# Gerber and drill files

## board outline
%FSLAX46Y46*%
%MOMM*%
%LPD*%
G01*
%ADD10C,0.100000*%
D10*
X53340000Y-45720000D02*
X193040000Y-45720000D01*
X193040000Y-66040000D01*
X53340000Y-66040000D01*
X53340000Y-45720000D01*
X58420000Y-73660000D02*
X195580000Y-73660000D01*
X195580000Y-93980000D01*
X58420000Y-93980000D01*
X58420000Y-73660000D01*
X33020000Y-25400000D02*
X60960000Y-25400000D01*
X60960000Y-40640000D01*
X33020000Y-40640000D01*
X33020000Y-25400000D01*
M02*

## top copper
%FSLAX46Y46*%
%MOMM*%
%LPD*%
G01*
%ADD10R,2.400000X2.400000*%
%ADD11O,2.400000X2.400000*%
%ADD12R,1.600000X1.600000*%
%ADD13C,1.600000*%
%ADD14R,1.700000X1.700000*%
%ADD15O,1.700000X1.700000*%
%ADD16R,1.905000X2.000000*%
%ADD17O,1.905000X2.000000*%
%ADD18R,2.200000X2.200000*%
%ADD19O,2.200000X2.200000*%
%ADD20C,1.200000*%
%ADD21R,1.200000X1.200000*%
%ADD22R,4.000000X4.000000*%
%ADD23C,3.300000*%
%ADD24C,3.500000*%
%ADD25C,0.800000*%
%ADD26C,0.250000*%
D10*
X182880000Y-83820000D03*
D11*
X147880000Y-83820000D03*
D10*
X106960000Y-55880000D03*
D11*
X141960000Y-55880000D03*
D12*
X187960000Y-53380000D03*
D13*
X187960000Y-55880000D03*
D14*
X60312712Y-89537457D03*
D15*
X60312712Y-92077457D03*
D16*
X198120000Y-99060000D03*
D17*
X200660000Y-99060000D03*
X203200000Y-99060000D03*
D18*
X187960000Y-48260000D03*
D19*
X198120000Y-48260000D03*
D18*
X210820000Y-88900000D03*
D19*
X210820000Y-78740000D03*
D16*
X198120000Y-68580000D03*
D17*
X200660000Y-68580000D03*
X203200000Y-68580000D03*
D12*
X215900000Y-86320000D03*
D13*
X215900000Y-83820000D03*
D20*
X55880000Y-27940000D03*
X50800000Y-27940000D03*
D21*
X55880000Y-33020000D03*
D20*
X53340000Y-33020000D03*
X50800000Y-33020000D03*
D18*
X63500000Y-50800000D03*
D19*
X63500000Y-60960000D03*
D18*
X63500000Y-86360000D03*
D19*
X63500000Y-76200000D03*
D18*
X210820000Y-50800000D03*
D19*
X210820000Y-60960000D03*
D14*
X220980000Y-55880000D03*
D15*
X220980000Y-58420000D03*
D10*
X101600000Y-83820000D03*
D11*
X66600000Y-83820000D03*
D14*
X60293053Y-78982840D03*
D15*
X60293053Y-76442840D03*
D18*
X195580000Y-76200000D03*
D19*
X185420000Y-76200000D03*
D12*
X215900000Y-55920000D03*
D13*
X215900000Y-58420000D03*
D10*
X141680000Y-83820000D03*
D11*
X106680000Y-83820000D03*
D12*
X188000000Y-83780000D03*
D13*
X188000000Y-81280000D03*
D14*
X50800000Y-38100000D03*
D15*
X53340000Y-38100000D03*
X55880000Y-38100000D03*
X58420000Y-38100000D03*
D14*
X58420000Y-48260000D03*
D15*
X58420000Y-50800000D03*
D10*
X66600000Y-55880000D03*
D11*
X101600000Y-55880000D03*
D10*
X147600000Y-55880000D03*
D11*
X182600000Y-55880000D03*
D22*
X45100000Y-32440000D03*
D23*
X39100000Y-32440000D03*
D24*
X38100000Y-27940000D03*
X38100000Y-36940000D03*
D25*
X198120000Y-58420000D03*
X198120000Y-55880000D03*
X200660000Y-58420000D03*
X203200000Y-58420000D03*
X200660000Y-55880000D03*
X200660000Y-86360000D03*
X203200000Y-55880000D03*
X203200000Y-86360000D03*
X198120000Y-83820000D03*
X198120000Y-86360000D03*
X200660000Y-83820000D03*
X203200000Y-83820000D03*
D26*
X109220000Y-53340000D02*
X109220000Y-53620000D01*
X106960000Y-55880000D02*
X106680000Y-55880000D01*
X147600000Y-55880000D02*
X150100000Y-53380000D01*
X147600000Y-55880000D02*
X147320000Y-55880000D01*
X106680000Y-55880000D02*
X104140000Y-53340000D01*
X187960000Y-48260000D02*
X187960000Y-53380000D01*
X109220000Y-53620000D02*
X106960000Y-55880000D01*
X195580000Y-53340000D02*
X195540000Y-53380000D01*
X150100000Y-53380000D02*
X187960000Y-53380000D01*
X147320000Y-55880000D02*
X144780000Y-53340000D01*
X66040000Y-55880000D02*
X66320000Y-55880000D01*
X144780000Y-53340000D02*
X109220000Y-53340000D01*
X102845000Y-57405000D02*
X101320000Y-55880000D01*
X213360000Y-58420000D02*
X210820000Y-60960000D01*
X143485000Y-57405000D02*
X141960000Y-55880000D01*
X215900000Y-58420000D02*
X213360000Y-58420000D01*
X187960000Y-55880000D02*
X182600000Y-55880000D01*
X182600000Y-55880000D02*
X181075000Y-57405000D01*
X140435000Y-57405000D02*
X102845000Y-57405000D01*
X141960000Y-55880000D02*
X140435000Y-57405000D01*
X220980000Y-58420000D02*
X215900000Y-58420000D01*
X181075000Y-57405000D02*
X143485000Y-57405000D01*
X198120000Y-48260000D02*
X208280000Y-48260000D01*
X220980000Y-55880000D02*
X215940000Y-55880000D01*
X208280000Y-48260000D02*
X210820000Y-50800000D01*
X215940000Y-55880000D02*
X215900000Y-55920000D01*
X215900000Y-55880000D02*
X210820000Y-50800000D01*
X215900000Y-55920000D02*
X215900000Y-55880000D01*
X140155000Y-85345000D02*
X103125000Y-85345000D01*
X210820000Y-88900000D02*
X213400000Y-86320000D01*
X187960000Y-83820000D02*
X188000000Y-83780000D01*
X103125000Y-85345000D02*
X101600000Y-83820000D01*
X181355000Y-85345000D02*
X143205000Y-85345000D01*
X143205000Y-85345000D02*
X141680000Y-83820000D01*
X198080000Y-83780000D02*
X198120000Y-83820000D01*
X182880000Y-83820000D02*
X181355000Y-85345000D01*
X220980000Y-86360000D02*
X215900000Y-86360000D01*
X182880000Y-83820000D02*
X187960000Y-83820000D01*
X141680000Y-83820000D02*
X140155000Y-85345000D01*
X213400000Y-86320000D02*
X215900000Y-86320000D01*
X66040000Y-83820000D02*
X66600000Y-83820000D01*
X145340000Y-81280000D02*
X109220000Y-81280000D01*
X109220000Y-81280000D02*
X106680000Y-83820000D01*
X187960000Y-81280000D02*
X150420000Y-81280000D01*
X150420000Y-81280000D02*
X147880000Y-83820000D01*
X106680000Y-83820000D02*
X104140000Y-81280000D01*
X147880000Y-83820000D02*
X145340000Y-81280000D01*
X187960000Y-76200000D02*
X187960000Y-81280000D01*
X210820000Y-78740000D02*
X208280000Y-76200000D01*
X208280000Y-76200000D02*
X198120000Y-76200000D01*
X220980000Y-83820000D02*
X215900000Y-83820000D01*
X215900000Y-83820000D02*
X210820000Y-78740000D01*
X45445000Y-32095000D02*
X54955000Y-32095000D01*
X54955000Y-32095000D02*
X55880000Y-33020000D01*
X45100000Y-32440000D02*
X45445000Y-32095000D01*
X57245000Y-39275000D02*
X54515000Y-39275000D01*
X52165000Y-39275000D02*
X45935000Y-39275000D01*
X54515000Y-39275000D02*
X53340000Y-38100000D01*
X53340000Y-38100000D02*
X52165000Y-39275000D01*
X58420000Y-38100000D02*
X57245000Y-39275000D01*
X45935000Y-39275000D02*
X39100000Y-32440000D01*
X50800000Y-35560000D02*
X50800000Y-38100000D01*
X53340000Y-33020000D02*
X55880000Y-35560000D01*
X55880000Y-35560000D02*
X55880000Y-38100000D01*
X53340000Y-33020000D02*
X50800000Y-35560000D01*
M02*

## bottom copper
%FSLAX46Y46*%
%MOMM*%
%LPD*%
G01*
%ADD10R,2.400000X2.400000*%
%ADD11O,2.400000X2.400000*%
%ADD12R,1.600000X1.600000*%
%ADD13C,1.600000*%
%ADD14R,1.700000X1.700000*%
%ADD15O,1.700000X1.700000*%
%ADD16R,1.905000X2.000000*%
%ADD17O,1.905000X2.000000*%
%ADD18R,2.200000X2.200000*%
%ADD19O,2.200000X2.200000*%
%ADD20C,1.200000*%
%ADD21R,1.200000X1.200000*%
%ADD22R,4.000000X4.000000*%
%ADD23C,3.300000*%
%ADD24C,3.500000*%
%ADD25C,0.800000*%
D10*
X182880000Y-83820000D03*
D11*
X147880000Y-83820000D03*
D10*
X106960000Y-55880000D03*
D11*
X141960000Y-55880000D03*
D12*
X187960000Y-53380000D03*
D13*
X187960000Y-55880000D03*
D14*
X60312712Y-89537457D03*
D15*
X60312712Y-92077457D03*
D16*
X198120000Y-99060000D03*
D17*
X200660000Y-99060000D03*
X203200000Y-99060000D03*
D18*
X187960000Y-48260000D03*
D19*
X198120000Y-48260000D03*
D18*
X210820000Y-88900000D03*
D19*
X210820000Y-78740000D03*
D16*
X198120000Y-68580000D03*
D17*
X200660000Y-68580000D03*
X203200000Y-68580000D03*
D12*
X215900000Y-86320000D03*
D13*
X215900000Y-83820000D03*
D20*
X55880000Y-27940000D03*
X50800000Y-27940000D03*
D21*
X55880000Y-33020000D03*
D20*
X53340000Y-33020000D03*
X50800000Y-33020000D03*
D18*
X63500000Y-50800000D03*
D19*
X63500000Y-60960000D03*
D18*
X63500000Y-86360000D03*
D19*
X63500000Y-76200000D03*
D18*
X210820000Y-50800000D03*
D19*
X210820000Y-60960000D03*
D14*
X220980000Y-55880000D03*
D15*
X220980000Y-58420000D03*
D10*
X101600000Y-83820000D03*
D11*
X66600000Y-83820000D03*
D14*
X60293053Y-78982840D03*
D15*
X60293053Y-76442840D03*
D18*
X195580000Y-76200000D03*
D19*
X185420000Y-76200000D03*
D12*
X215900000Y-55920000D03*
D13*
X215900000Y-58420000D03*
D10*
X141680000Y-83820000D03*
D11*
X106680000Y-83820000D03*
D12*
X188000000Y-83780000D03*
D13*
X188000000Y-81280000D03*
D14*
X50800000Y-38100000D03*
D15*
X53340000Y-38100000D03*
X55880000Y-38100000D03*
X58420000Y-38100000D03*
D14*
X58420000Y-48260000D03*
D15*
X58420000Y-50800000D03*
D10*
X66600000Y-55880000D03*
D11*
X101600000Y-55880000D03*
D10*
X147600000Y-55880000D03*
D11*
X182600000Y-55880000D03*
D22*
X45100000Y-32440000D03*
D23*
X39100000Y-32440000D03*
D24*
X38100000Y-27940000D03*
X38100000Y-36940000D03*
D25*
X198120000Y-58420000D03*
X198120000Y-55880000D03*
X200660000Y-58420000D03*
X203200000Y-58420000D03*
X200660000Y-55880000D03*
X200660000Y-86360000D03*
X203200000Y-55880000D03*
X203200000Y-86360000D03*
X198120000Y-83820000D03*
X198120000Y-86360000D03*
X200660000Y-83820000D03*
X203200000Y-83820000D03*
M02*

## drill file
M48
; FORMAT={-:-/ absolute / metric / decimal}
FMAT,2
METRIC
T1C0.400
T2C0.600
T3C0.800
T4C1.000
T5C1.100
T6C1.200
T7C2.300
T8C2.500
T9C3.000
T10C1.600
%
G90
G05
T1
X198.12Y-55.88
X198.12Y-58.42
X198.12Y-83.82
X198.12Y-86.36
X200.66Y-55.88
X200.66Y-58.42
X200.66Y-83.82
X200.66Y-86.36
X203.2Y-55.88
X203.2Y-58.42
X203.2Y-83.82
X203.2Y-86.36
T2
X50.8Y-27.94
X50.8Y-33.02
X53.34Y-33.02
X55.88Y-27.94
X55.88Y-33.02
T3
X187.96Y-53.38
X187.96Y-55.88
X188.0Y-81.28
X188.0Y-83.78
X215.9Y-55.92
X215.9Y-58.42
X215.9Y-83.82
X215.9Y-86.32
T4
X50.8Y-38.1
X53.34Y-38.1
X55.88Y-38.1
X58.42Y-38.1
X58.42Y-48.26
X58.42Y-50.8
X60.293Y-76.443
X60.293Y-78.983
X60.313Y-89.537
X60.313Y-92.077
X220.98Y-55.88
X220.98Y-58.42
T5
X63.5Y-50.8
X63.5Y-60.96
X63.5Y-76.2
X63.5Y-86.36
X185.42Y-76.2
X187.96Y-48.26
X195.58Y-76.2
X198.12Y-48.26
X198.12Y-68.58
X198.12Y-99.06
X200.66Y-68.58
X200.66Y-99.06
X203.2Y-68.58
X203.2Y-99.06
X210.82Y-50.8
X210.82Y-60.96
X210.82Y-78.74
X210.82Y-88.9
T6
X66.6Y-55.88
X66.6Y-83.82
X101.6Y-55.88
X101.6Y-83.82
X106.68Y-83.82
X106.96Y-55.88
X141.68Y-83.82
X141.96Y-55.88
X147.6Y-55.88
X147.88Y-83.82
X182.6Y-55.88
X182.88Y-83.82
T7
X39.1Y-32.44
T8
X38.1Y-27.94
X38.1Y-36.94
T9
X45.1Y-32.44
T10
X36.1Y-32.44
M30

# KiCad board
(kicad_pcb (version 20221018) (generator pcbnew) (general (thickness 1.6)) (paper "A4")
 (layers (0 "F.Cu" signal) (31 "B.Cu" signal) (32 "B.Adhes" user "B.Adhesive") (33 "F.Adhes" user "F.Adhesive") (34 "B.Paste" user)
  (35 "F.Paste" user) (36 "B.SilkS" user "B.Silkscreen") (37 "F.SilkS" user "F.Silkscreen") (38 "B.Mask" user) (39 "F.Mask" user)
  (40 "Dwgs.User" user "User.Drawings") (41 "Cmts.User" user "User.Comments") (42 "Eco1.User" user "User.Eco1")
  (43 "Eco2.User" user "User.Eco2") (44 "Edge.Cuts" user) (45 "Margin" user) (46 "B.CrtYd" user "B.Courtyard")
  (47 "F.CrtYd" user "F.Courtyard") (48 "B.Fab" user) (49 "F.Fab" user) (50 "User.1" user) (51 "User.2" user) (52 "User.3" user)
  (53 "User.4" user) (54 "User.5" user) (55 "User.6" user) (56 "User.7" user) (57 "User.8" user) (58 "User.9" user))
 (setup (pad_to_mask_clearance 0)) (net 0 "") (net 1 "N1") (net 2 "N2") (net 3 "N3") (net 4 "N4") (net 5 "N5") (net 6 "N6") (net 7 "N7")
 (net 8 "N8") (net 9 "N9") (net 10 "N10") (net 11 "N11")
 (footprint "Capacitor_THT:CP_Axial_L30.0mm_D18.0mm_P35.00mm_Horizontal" (layer "F.Cu") (at 182.88 83.82 180)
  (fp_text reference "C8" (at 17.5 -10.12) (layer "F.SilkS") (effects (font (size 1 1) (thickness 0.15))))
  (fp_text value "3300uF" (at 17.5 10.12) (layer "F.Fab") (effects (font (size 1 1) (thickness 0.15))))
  (pad "1" thru_hole rect (at 0 0 180) (size 2.4 2.4) (drill 1.2) (layers "*.Cu" "*.Mask") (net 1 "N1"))
  (pad "2" thru_hole oval (at 35 0 180) (size 2.4 2.4) (drill 1.2) (layers "*.Cu" "*.Mask") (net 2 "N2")))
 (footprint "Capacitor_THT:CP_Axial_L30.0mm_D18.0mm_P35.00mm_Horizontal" (layer "F.Cu") (at 106.96 55.88)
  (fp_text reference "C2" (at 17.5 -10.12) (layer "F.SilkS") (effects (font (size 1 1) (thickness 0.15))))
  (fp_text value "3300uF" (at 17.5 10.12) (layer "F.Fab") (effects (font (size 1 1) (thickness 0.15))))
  (pad "1" thru_hole rect (at 0 0) (size 2.4 2.4) (drill 1.2) (layers "*.Cu" "*.Mask") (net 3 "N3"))
  (pad "2" thru_hole oval (at 35 0) (size 2.4 2.4) (drill 1.2) (layers "*.Cu" "*.Mask") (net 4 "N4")))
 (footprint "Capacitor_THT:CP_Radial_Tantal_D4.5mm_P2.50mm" (layer "F.Cu") (at 187.96 53.38 -90)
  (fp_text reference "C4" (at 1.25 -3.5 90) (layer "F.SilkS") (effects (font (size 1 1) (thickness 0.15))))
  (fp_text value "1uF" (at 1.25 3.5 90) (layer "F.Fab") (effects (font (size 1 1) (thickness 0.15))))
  (pad "1" thru_hole rect (at 0 0 270) (size 1.6 1.6) (drill 0.8) (layers "*.Cu" "*.Mask") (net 3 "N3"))
  (pad "2" thru_hole circle (at 2.5 0 270) (size 1.6 1.6) (drill 0.8) (layers "*.Cu" "*.Mask") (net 4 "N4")))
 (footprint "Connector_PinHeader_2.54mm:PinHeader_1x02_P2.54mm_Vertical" (layer "F.Cu") (at 60.312712 89.537457)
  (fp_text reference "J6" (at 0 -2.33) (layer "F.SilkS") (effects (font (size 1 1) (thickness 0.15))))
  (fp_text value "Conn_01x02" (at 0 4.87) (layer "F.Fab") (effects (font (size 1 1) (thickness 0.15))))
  (pad "1" thru_hole rect (at 0 0) (size 1.7 1.7) (drill 1) (layers "*.Cu" "*.Mask") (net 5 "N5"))
  (pad "2" thru_hole oval (at 0 2.54) (size 1.7 1.7) (drill 1) (layers "*.Cu" "*.Mask") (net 1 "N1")))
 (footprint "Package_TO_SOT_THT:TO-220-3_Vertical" (layer "F.Cu") (at 198.12 99.06)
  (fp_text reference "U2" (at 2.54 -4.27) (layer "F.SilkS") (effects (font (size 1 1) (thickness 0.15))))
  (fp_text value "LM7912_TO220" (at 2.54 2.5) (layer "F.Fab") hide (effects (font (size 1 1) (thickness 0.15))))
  (pad "1" thru_hole rect (at 0 0) (size 1.905 2) (drill 1.1) (layers "*.Cu" "*.Mask") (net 1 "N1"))
  (pad "2" thru_hole oval (at 2.54 0) (size 1.905 2) (drill 1.1) (layers "*.Cu" "*.Mask") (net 2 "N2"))
  (pad "3" thru_hole oval (at 5.08 0) (size 1.905 2) (drill 1.1) (layers "*.Cu" "*.Mask") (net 5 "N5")))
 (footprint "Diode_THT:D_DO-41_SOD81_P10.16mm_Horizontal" (layer "F.Cu") (at 187.96 48.26)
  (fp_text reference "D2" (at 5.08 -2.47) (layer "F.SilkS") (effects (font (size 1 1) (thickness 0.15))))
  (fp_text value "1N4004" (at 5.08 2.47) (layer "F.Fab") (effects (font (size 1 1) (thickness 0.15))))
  (pad "1" thru_hole rect (at 0 0) (size 2.2 2.2) (drill 1.1) (layers "*.Cu" "*.Mask") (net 3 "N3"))
  (pad "2" thru_hole oval (at 10.16 0) (size 2.2 2.2) (drill 1.1) (layers "*.Cu" "*.Mask") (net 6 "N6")))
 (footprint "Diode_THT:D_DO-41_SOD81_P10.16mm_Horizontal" (layer "F.Cu") (at 210.82 88.9 90)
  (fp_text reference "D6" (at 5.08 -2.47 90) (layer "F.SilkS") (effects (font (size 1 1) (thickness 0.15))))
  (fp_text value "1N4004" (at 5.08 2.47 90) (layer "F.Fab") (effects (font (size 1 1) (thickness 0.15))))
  (pad "1" thru_hole rect (at 0 0 90) (size 2.2 2.2) (drill 1.1) (layers "*.Cu" "*.Mask") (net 1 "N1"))
  (pad "2" thru_hole oval (at 10.16 0 90) (size 2.2 2.2) (drill 1.1) (layers "*.Cu" "*.Mask") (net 5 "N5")))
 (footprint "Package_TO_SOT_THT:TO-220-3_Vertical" (layer "F.Cu") (at 198.12 68.58)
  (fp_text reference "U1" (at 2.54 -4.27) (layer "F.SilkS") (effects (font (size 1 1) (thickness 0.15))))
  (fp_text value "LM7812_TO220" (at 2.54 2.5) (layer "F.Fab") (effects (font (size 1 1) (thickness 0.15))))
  (pad "1" thru_hole rect (at 0 0) (size 1.905 2) (drill 1.1) (layers "*.Cu" "*.Mask") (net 3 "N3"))
  (pad "2" thru_hole oval (at 2.54 0) (size 1.905 2) (drill 1.1) (layers "*.Cu" "*.Mask") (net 4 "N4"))
  (pad "3" thru_hole oval (at 5.08 0) (size 1.905 2) (drill 1.1) (layers "*.Cu" "*.Mask") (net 6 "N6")))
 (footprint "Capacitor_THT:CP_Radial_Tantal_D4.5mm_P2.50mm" (layer "F.Cu") (at 215.9 86.32 90)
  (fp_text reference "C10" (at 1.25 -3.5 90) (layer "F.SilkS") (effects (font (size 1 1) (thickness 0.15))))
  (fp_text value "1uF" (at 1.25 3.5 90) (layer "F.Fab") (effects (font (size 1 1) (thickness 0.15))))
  (pad "1" thru_hole rect (at 0 0 90) (size 1.6 1.6) (drill 0.8) (layers "*.Cu" "*.Mask") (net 1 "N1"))
  (pad "2" thru_hole circle (at 2.5 0 90) (size 1.6 1.6) (drill 0.8) (layers "*.Cu" "*.Mask") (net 5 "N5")))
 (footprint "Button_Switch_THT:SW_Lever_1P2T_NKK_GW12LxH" (layer "F.Cu") (at 55.88 33.02 180)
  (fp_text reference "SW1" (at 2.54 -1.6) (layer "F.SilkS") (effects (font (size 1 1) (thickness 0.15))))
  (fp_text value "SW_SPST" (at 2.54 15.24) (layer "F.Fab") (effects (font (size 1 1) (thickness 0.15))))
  (pad "" thru_hole circle (at 0 5.08 180) (size 1.2 1.2) (drill 0.6) (layers "*.Cu" "*.Mask"))
  (pad "" thru_hole circle (at 5.08 5.08 180) (size 1.2 1.2) (drill 0.6) (layers "*.Cu" "*.Mask"))
  (pad "1" thru_hole rect (at 0 0 180) (size 1.2 1.2) (drill 0.6) (layers "*.Cu" "*.Mask") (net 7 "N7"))
  (pad "2" thru_hole circle (at 2.54 0 180) (size 1.2 1.2) (drill 0.6) (layers "*.Cu" "*.Mask") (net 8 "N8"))
  (pad "3" thru_hole circle (at 5.08 0 180) (size 1.2 1.2) (drill 0.6) (layers "*.Cu" "*.Mask")))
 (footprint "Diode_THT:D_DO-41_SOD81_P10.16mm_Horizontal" (layer "F.Cu") (at 63.5 50.8 -90)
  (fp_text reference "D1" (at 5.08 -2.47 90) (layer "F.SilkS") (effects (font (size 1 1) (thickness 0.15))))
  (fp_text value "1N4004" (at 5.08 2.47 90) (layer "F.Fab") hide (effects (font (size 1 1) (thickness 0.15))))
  (pad "1" thru_hole rect (at 0 0 270) (size 2.2 2.2) (drill 1.1) (layers "*.Cu" "*.Mask") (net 3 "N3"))
  (pad "2" thru_hole oval (at 10.16 0 270) (size 2.2 2.2) (drill 1.1) (layers "*.Cu" "*.Mask") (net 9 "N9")))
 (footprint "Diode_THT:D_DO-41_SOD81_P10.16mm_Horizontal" (layer "F.Cu") (at 63.5 86.36 90)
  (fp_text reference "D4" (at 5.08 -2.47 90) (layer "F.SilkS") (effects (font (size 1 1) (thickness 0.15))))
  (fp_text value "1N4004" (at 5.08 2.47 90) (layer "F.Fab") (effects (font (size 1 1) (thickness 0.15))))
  (pad "1" thru_hole rect (at 0 0 90) (size 2.2 2.2) (drill 1.1) (layers "*.Cu" "*.Mask") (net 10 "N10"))
  (pad "2" thru_hole oval (at 10.16 0 90) (size 2.2 2.2) (drill 1.1) (layers "*.Cu" "*.Mask") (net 2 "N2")))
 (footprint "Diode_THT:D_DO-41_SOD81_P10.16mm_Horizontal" (layer "F.Cu") (at 210.82 50.8 -90)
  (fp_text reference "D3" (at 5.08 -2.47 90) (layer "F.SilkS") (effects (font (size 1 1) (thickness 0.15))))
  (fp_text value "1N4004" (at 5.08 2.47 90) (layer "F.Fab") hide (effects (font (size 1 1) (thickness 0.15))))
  (pad "1" thru_hole rect (at 0 0 270) (size 2.2 2.2) (drill 1.1) (layers "*.Cu" "*.Mask") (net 6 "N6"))
  (pad "2" thru_hole oval (at 10.16 0 270) (size 2.2 2.2) (drill 1.1) (layers "*.Cu" "*.Mask") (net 4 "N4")))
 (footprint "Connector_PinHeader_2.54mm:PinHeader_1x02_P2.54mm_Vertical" (layer "F.Cu") (at 220.98 55.88)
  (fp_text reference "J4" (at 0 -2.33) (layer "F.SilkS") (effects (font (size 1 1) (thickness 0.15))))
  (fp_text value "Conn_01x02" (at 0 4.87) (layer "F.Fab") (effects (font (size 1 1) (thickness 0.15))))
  (pad "1" thru_hole rect (at 0 0) (size 1.7 1.7) (drill 1) (layers "*.Cu" "*.Mask") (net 6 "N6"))
  (pad "2" thru_hole oval (at 0 2.54) (size 1.7 1.7) (drill 1) (layers "*.Cu" "*.Mask") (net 4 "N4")))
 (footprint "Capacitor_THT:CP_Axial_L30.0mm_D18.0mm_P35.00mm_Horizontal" (layer "F.Cu") (at 101.6 83.82 180)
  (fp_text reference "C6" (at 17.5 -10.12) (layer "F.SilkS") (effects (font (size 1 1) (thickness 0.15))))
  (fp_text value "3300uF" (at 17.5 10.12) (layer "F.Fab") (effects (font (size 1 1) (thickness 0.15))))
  (pad "1" thru_hole rect (at 0 0 180) (size 2.4 2.4) (drill 1.2) (layers "*.Cu" "*.Mask") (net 1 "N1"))
  (pad "2" thru_hole oval (at 35 0 180) (size 2.4 2.4) (drill 1.2) (layers "*.Cu" "*.Mask") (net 2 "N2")))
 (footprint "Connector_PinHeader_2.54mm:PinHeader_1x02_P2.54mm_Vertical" (layer "F.Cu") (at 60.293053 78.98284 180)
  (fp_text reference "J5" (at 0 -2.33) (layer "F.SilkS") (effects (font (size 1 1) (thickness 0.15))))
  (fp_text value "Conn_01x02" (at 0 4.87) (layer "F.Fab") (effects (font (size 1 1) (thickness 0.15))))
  (pad "1" thru_hole rect (at 0 0 180) (size 1.7 1.7) (drill 1) (layers "*.Cu" "*.Mask") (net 1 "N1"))
  (pad "2" thru_hole oval (at 0 2.54 180) (size 1.7 1.7) (drill 1) (layers "*.Cu" "*.Mask") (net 10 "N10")))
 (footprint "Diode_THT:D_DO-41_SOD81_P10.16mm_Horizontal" (layer "F.Cu") (at 195.58 76.2 180)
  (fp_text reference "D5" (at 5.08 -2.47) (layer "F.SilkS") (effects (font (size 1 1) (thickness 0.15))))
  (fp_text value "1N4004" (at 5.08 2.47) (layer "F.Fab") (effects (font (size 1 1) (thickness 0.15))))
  (pad "1" thru_hole rect (at 0 0 180) (size 2.2 2.2) (drill 1.1) (layers "*.Cu" "*.Mask") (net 5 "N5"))
  (pad "2" thru_hole oval (at 10.16 0 180) (size 2.2 2.2) (drill 1.1) (layers "*.Cu" "*.Mask") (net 2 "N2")))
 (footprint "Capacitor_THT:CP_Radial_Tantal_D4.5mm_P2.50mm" (layer "F.Cu") (at 215.9 55.92 -90)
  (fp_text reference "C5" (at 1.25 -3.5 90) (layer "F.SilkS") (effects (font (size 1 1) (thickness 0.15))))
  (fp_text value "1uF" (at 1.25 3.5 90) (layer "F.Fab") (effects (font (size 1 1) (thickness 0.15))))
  (pad "1" thru_hole rect (at 0 0 270) (size 1.6 1.6) (drill 0.8) (layers "*.Cu" "*.Mask") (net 6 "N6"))
  (pad "2" thru_hole circle (at 2.5 0 270) (size 1.6 1.6) (drill 0.8) (layers "*.Cu" "*.Mask") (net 4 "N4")))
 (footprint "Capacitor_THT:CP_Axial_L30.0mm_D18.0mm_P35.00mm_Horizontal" (layer "F.Cu") (at 141.68 83.82 180)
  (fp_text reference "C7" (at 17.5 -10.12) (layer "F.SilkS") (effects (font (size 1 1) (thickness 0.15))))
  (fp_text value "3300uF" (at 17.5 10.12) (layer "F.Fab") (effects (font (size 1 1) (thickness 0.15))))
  (pad "1" thru_hole rect (at 0 0 180) (size 2.4 2.4) (drill 1.2) (layers "*.Cu" "*.Mask") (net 1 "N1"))
  (pad "2" thru_hole oval (at 35 0 180) (size 2.4 2.4) (drill 1.2) (layers "*.Cu" "*.Mask") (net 2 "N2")))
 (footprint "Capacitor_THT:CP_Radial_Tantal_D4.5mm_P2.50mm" (layer "F.Cu") (at 188 83.78 90)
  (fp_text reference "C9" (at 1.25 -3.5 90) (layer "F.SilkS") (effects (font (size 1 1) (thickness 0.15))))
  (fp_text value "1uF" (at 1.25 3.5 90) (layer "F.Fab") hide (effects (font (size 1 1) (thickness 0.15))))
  (pad "1" thru_hole rect (at 0 0 90) (size 1.6 1.6) (drill 0.8) (layers "*.Cu" "*.Mask") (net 1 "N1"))
  (pad "2" thru_hole circle (at 2.5 0 90) (size 1.6 1.6) (drill 0.8) (layers "*.Cu" "*.Mask") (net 2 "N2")))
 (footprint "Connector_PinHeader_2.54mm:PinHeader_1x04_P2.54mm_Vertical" (layer "F.Cu") (at 50.8 38.1 90)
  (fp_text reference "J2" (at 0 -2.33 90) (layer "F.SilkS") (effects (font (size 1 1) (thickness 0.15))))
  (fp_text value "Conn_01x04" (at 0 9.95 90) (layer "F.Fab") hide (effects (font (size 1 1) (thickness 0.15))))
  (pad "1" thru_hole rect (at 0 0 90) (size 1.7 1.7) (drill 1) (layers "*.Cu" "*.Mask") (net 8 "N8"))
  (pad "2" thru_hole oval (at 0 2.54 90) (size 1.7 1.7) (drill 1) (layers "*.Cu" "*.Mask") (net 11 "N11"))
  (pad "3" thru_hole oval (at 0 5.08 90) (size 1.7 1.7) (drill 1) (layers "*.Cu" "*.Mask") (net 8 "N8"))
  (pad "4" thru_hole oval (at 0 7.62 90) (size 1.7 1.7) (drill 1) (layers "*.Cu" "*.Mask") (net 11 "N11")))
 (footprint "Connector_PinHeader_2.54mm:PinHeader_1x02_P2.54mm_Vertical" (layer "F.Cu") (at 58.42 48.26)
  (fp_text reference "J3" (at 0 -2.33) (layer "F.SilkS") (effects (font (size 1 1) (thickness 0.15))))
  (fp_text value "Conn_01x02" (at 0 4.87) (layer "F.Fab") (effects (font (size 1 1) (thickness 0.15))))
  (pad "1" thru_hole rect (at 0 0) (size 1.7 1.7) (drill 1) (layers "*.Cu" "*.Mask") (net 4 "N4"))
  (pad "2" thru_hole oval (at 0 2.54) (size 1.7 1.7) (drill 1) (layers "*.Cu" "*.Mask") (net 9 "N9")))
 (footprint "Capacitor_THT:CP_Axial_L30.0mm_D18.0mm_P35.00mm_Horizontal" (layer "F.Cu") (at 66.6 55.88)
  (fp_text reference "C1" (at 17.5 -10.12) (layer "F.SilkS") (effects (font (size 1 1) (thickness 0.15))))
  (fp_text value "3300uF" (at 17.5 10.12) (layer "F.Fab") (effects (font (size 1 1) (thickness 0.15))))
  (pad "1" thru_hole rect (at 0 0) (size 2.4 2.4) (drill 1.2) (layers "*.Cu" "*.Mask") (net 3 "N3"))
  (pad "2" thru_hole oval (at 35 0) (size 2.4 2.4) (drill 1.2) (layers "*.Cu" "*.Mask") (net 4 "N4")))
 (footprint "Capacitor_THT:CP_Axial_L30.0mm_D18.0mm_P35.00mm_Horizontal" (layer "F.Cu") (at 147.6 55.88)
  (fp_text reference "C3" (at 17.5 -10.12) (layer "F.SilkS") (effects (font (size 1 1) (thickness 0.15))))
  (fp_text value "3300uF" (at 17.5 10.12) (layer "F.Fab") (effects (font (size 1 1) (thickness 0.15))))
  (pad "1" thru_hole rect (at 0 0) (size 2.4 2.4) (drill 1.2) (layers "*.Cu" "*.Mask") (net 3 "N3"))
  (pad "2" thru_hole oval (at 35 0) (size 2.4 2.4) (drill 1.2) (layers "*.Cu" "*.Mask") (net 4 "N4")))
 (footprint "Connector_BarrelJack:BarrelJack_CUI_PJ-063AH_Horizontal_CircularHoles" (layer "F.Cu") (at 45.1 32.44 -90)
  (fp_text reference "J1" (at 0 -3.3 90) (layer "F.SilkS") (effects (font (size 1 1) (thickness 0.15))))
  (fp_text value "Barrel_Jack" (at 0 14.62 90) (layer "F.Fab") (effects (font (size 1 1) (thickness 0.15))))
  (pad "" np_thru_hole circle (at 0 9 270) (size 1.6 1.6) (drill 1.6) (layers "*.Cu" "*.Mask"))
  (pad "1" thru_hole rect (at 0 0 270) (size 4 4) (drill 3) (layers "*.Cu" "*.Mask") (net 7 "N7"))
  (pad "2" thru_hole circle (at 0 6 270) (size 3.3 3.3) (drill 2.3) (layers "*.Cu" "*.Mask") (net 11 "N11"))
  (pad "MP" thru_hole circle (at -4.5 7 270) (size 3.5 3.5) (drill 2.5) (layers "*.Cu" "*.Mask"))
  (pad "MP" thru_hole circle (at 4.5 7 270) (size 3.5 3.5) (drill 2.5) (layers "*.Cu" "*.Mask")))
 (gr_rect (start 53.34 45.72) (end 193.04 66.04) (stroke (width 0.1) (type default)) (fill none) (layer "Edge.Cuts"))
 (gr_rect (start 58.42 73.66) (end 195.58 93.98) (stroke (width 0.1) (type default)) (fill none) (layer "Edge.Cuts"))
 (gr_rect (start 33.02 25.4) (end 60.96 40.64) (stroke (width 0.1) (type default)) (fill none) (layer "Edge.Cuts"))
 (segment (start 109.22 53.34) (end 109.22 53.62) (width 0.25) (layer "F.Cu") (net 3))
 (segment (start 106.96 55.88) (end 106.68 55.88) (width 0.25) (layer "F.Cu") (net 3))
 (segment (start 147.6 55.88) (end 150.1 53.38) (width 0.25) (layer "F.Cu") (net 3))
 (segment (start 147.6 55.88) (end 147.32 55.88) (width 0.25) (layer "F.Cu") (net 3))
 (segment (start 106.68 55.88) (end 104.14 53.34) (width 0.25) (layer "F.Cu") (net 3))
 (segment (start 187.96 48.26) (end 187.96 53.38) (width 0.25) (layer "F.Cu") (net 3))
 (segment (start 109.22 53.62) (end 106.96 55.88) (width 0.25) (layer "F.Cu") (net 3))
 (segment (start 195.58 53.34) (end 195.54 53.38) (width 0.25) (layer "F.Cu") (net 3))
 (segment (start 150.1 53.38) (end 187.96 53.38) (width 0.25) (layer "F.Cu") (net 3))
 (segment (start 147.32 55.88) (end 144.78 53.34) (width 0.25) (layer "F.Cu") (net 3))
 (segment (start 66.04 55.88) (end 66.32 55.88) (width 0.25) (layer "F.Cu") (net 3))
 (segment (start 144.78 53.34) (end 109.22 53.34) (width 0.25) (layer "F.Cu") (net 3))
 (via (at 198.12 58.42) (size 0.8) (drill 0.4) (layers "F.Cu" "B.Cu") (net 3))
 (via (at 198.12 55.88) (size 0.8) (drill 0.4) (layers "F.Cu" "B.Cu") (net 3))
 (segment (start 102.845 57.405) (end 101.32 55.88) (width 0.25) (layer "F.Cu") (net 4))
 (segment (start 213.36 58.42) (end 210.82 60.96) (width 0.25) (layer "F.Cu") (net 4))
 (segment (start 143.485 57.405) (end 141.96 55.88) (width 0.25) (layer "F.Cu") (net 4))
 (segment (start 215.9 58.42) (end 213.36 58.42) (width 0.25) (layer "F.Cu") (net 4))
 (segment (start 187.96 55.88) (end 182.6 55.88) (width 0.25) (layer "F.Cu") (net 4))
 (segment (start 182.6 55.88) (end 181.075 57.405) (width 0.25) (layer "F.Cu") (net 4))
 (segment (start 140.435 57.405) (end 102.845 57.405) (width 0.25) (layer "F.Cu") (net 4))
 (segment (start 141.96 55.88) (end 140.435 57.405) (width 0.25) (layer "F.Cu") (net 4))
 (segment (start 220.98 58.42) (end 215.9 58.42) (width 0.25) (layer "F.Cu") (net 4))
 (segment (start 181.075 57.405) (end 143.485 57.405) (width 0.25) (layer "F.Cu") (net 4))
 (via (at 200.66 58.42) (size 0.8) (drill 0.4) (layers "F.Cu" "B.Cu") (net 4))
 (via (at 203.2 58.42) (size 0.8) (drill 0.4) (layers "F.Cu" "B.Cu") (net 4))
 (via (at 200.66 55.88) (size 0.8) (drill 0.4) (layers "F.Cu" "B.Cu") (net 4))
 (via (at 200.66 86.36) (size 0.8) (drill 0.4) (layers "F.Cu" "B.Cu") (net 4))
 (segment (start 198.12 48.26) (end 208.28 48.26) (width 0.25) (layer "F.Cu") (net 6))
 (segment (start 220.98 55.88) (end 215.94 55.88) (width 0.25) (layer "F.Cu") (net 6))
 (segment (start 208.28 48.26) (end 210.82 50.8) (width 0.25) (layer "F.Cu") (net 6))
 (segment (start 215.94 55.88) (end 215.9 55.92) (width 0.25) (layer "F.Cu") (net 6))
 (segment (start 215.9 55.88) (end 210.82 50.8) (width 0.25) (layer "F.Cu") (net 6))
 (segment (start 215.9 55.92) (end 215.9 55.88) (width 0.25) (layer "F.Cu") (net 6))
 (via (at 203.2 55.88) (size 0.8) (drill 0.4) (layers "F.Cu" "B.Cu") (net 6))
 (via (at 203.2 86.36) (size 0.8) (drill 0.4) (layers "F.Cu" "B.Cu") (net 6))
 (segment (start 140.155 85.345) (end 103.125 85.345) (width 0.25) (layer "F.Cu") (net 1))
 (segment (start 210.82 88.9) (end 213.4 86.32) (width 0.25) (layer "F.Cu") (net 1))
 (segment (start 187.96 83.82) (end 188 83.78) (width 0.25) (layer "F.Cu") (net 1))
 (segment (start 103.125 85.345) (end 101.6 83.82) (width 0.25) (layer "F.Cu") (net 1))
 (segment (start 181.355 85.345) (end 143.205 85.345) (width 0.25) (layer "F.Cu") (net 1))
 (segment (start 143.205 85.345) (end 141.68 83.82) (width 0.25) (layer "F.Cu") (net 1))
 (segment (start 198.08 83.78) (end 198.12 83.82) (width 0.25) (layer "F.Cu") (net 1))
 (segment (start 182.88 83.82) (end 181.355 85.345) (width 0.25) (layer "F.Cu") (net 1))
 (segment (start 220.98 86.36) (end 215.9 86.36) (width 0.25) (layer "F.Cu") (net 1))
 (segment (start 182.88 83.82) (end 187.96 83.82) (width 0.25) (layer "F.Cu") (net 1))
 (segment (start 141.68 83.82) (end 140.155 85.345) (width 0.25) (layer "F.Cu") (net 1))
 (segment (start 213.4 86.32) (end 215.9 86.32) (width 0.25) (layer "F.Cu") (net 1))
 (via (at 198.12 83.82) (size 0.8) (drill 0.4) (layers "F.Cu" "B.Cu") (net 1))
 (via (at 198.12 86.36) (size 0.8) (drill 0.4) (layers "F.Cu" "B.Cu") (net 1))
 (segment (start 66.04 83.82) (end 66.6 83.82) (width 0.25) (layer "F.Cu") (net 2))
 (segment (start 145.34 81.28) (end 109.22 81.28) (width 0.25) (layer "F.Cu") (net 2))
 (segment (start 109.22 81.28) (end 106.68 83.82) (width 0.25) (layer "F.Cu") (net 2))
 (segment (start 187.96 81.28) (end 150.42 81.28) (width 0.25) (layer "F.Cu") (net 2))
 (segment (start 150.42 81.28) (end 147.88 83.82) (width 0.25) (layer "F.Cu") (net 2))
 (segment (start 106.68 83.82) (end 104.14 81.28) (width 0.25) (layer "F.Cu") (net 2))
 (segment (start 147.88 83.82) (end 145.34 81.28) (width 0.25) (layer "F.Cu") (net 2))
 (segment (start 187.96 76.2) (end 187.96 81.28) (width 0.25) (layer "F.Cu") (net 2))
 (via (at 200.66 83.82) (size 0.8) (drill 0.4) (layers "F.Cu" "B.Cu") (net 2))
 (segment (start 210.82 78.74) (end 208.28 76.2) (width 0.25) (layer "F.Cu") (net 5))
 (segment (start 208.28 76.2) (end 198.12 76.2) (width 0.25) (layer "F.Cu") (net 5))
 (segment (start 220.98 83.82) (end 215.9 83.82) (width 0.25) (layer "F.Cu") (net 5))
 (segment (start 215.9 83.82) (end 210.82 78.74) (width 0.25) (layer "F.Cu") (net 5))
 (via (at 203.2 83.82) (size 0.8) (drill 0.4) (layers "F.Cu" "B.Cu") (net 5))
 (segment (start 45.445 32.095) (end 54.955 32.095) (width 0.25) (layer "F.Cu") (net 7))
 (segment (start 54.955 32.095) (end 55.88 33.02) (width 0.25) (layer "F.Cu") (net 7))
 (segment (start 45.1 32.44) (end 45.445 32.095) (width 0.25) (layer "F.Cu") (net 7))
 (segment (start 57.245 39.275) (end 54.515 39.275) (width 0.25) (layer "F.Cu") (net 11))
 (segment (start 52.165 39.275) (end 45.935 39.275) (width 0.25) (layer "F.Cu") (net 11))
 (segment (start 54.515 39.275) (end 53.34 38.1) (width 0.25) (layer "F.Cu") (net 11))
 (segment (start 53.34 38.1) (end 52.165 39.275) (width 0.25) (layer "F.Cu") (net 11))
 (segment (start 58.42 38.1) (end 57.245 39.275) (width 0.25) (layer "F.Cu") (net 11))
 (segment (start 45.935 39.275) (end 39.1 32.44) (width 0.25) (layer "F.Cu") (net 11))
 (segment (start 50.8 35.56) (end 50.8 38.1) (width 0.25) (layer "F.Cu") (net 8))
 (segment (start 53.34 33.02) (end 55.88 35.56) (width 0.25) (layer "F.Cu") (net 8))
 (segment (start 55.88 35.56) (end 55.88 38.1) (width 0.25) (layer "F.Cu") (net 8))
 (segment (start 53.34 33.02) (end 50.8 35.56) (width 0.25) (layer "F.Cu") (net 8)))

